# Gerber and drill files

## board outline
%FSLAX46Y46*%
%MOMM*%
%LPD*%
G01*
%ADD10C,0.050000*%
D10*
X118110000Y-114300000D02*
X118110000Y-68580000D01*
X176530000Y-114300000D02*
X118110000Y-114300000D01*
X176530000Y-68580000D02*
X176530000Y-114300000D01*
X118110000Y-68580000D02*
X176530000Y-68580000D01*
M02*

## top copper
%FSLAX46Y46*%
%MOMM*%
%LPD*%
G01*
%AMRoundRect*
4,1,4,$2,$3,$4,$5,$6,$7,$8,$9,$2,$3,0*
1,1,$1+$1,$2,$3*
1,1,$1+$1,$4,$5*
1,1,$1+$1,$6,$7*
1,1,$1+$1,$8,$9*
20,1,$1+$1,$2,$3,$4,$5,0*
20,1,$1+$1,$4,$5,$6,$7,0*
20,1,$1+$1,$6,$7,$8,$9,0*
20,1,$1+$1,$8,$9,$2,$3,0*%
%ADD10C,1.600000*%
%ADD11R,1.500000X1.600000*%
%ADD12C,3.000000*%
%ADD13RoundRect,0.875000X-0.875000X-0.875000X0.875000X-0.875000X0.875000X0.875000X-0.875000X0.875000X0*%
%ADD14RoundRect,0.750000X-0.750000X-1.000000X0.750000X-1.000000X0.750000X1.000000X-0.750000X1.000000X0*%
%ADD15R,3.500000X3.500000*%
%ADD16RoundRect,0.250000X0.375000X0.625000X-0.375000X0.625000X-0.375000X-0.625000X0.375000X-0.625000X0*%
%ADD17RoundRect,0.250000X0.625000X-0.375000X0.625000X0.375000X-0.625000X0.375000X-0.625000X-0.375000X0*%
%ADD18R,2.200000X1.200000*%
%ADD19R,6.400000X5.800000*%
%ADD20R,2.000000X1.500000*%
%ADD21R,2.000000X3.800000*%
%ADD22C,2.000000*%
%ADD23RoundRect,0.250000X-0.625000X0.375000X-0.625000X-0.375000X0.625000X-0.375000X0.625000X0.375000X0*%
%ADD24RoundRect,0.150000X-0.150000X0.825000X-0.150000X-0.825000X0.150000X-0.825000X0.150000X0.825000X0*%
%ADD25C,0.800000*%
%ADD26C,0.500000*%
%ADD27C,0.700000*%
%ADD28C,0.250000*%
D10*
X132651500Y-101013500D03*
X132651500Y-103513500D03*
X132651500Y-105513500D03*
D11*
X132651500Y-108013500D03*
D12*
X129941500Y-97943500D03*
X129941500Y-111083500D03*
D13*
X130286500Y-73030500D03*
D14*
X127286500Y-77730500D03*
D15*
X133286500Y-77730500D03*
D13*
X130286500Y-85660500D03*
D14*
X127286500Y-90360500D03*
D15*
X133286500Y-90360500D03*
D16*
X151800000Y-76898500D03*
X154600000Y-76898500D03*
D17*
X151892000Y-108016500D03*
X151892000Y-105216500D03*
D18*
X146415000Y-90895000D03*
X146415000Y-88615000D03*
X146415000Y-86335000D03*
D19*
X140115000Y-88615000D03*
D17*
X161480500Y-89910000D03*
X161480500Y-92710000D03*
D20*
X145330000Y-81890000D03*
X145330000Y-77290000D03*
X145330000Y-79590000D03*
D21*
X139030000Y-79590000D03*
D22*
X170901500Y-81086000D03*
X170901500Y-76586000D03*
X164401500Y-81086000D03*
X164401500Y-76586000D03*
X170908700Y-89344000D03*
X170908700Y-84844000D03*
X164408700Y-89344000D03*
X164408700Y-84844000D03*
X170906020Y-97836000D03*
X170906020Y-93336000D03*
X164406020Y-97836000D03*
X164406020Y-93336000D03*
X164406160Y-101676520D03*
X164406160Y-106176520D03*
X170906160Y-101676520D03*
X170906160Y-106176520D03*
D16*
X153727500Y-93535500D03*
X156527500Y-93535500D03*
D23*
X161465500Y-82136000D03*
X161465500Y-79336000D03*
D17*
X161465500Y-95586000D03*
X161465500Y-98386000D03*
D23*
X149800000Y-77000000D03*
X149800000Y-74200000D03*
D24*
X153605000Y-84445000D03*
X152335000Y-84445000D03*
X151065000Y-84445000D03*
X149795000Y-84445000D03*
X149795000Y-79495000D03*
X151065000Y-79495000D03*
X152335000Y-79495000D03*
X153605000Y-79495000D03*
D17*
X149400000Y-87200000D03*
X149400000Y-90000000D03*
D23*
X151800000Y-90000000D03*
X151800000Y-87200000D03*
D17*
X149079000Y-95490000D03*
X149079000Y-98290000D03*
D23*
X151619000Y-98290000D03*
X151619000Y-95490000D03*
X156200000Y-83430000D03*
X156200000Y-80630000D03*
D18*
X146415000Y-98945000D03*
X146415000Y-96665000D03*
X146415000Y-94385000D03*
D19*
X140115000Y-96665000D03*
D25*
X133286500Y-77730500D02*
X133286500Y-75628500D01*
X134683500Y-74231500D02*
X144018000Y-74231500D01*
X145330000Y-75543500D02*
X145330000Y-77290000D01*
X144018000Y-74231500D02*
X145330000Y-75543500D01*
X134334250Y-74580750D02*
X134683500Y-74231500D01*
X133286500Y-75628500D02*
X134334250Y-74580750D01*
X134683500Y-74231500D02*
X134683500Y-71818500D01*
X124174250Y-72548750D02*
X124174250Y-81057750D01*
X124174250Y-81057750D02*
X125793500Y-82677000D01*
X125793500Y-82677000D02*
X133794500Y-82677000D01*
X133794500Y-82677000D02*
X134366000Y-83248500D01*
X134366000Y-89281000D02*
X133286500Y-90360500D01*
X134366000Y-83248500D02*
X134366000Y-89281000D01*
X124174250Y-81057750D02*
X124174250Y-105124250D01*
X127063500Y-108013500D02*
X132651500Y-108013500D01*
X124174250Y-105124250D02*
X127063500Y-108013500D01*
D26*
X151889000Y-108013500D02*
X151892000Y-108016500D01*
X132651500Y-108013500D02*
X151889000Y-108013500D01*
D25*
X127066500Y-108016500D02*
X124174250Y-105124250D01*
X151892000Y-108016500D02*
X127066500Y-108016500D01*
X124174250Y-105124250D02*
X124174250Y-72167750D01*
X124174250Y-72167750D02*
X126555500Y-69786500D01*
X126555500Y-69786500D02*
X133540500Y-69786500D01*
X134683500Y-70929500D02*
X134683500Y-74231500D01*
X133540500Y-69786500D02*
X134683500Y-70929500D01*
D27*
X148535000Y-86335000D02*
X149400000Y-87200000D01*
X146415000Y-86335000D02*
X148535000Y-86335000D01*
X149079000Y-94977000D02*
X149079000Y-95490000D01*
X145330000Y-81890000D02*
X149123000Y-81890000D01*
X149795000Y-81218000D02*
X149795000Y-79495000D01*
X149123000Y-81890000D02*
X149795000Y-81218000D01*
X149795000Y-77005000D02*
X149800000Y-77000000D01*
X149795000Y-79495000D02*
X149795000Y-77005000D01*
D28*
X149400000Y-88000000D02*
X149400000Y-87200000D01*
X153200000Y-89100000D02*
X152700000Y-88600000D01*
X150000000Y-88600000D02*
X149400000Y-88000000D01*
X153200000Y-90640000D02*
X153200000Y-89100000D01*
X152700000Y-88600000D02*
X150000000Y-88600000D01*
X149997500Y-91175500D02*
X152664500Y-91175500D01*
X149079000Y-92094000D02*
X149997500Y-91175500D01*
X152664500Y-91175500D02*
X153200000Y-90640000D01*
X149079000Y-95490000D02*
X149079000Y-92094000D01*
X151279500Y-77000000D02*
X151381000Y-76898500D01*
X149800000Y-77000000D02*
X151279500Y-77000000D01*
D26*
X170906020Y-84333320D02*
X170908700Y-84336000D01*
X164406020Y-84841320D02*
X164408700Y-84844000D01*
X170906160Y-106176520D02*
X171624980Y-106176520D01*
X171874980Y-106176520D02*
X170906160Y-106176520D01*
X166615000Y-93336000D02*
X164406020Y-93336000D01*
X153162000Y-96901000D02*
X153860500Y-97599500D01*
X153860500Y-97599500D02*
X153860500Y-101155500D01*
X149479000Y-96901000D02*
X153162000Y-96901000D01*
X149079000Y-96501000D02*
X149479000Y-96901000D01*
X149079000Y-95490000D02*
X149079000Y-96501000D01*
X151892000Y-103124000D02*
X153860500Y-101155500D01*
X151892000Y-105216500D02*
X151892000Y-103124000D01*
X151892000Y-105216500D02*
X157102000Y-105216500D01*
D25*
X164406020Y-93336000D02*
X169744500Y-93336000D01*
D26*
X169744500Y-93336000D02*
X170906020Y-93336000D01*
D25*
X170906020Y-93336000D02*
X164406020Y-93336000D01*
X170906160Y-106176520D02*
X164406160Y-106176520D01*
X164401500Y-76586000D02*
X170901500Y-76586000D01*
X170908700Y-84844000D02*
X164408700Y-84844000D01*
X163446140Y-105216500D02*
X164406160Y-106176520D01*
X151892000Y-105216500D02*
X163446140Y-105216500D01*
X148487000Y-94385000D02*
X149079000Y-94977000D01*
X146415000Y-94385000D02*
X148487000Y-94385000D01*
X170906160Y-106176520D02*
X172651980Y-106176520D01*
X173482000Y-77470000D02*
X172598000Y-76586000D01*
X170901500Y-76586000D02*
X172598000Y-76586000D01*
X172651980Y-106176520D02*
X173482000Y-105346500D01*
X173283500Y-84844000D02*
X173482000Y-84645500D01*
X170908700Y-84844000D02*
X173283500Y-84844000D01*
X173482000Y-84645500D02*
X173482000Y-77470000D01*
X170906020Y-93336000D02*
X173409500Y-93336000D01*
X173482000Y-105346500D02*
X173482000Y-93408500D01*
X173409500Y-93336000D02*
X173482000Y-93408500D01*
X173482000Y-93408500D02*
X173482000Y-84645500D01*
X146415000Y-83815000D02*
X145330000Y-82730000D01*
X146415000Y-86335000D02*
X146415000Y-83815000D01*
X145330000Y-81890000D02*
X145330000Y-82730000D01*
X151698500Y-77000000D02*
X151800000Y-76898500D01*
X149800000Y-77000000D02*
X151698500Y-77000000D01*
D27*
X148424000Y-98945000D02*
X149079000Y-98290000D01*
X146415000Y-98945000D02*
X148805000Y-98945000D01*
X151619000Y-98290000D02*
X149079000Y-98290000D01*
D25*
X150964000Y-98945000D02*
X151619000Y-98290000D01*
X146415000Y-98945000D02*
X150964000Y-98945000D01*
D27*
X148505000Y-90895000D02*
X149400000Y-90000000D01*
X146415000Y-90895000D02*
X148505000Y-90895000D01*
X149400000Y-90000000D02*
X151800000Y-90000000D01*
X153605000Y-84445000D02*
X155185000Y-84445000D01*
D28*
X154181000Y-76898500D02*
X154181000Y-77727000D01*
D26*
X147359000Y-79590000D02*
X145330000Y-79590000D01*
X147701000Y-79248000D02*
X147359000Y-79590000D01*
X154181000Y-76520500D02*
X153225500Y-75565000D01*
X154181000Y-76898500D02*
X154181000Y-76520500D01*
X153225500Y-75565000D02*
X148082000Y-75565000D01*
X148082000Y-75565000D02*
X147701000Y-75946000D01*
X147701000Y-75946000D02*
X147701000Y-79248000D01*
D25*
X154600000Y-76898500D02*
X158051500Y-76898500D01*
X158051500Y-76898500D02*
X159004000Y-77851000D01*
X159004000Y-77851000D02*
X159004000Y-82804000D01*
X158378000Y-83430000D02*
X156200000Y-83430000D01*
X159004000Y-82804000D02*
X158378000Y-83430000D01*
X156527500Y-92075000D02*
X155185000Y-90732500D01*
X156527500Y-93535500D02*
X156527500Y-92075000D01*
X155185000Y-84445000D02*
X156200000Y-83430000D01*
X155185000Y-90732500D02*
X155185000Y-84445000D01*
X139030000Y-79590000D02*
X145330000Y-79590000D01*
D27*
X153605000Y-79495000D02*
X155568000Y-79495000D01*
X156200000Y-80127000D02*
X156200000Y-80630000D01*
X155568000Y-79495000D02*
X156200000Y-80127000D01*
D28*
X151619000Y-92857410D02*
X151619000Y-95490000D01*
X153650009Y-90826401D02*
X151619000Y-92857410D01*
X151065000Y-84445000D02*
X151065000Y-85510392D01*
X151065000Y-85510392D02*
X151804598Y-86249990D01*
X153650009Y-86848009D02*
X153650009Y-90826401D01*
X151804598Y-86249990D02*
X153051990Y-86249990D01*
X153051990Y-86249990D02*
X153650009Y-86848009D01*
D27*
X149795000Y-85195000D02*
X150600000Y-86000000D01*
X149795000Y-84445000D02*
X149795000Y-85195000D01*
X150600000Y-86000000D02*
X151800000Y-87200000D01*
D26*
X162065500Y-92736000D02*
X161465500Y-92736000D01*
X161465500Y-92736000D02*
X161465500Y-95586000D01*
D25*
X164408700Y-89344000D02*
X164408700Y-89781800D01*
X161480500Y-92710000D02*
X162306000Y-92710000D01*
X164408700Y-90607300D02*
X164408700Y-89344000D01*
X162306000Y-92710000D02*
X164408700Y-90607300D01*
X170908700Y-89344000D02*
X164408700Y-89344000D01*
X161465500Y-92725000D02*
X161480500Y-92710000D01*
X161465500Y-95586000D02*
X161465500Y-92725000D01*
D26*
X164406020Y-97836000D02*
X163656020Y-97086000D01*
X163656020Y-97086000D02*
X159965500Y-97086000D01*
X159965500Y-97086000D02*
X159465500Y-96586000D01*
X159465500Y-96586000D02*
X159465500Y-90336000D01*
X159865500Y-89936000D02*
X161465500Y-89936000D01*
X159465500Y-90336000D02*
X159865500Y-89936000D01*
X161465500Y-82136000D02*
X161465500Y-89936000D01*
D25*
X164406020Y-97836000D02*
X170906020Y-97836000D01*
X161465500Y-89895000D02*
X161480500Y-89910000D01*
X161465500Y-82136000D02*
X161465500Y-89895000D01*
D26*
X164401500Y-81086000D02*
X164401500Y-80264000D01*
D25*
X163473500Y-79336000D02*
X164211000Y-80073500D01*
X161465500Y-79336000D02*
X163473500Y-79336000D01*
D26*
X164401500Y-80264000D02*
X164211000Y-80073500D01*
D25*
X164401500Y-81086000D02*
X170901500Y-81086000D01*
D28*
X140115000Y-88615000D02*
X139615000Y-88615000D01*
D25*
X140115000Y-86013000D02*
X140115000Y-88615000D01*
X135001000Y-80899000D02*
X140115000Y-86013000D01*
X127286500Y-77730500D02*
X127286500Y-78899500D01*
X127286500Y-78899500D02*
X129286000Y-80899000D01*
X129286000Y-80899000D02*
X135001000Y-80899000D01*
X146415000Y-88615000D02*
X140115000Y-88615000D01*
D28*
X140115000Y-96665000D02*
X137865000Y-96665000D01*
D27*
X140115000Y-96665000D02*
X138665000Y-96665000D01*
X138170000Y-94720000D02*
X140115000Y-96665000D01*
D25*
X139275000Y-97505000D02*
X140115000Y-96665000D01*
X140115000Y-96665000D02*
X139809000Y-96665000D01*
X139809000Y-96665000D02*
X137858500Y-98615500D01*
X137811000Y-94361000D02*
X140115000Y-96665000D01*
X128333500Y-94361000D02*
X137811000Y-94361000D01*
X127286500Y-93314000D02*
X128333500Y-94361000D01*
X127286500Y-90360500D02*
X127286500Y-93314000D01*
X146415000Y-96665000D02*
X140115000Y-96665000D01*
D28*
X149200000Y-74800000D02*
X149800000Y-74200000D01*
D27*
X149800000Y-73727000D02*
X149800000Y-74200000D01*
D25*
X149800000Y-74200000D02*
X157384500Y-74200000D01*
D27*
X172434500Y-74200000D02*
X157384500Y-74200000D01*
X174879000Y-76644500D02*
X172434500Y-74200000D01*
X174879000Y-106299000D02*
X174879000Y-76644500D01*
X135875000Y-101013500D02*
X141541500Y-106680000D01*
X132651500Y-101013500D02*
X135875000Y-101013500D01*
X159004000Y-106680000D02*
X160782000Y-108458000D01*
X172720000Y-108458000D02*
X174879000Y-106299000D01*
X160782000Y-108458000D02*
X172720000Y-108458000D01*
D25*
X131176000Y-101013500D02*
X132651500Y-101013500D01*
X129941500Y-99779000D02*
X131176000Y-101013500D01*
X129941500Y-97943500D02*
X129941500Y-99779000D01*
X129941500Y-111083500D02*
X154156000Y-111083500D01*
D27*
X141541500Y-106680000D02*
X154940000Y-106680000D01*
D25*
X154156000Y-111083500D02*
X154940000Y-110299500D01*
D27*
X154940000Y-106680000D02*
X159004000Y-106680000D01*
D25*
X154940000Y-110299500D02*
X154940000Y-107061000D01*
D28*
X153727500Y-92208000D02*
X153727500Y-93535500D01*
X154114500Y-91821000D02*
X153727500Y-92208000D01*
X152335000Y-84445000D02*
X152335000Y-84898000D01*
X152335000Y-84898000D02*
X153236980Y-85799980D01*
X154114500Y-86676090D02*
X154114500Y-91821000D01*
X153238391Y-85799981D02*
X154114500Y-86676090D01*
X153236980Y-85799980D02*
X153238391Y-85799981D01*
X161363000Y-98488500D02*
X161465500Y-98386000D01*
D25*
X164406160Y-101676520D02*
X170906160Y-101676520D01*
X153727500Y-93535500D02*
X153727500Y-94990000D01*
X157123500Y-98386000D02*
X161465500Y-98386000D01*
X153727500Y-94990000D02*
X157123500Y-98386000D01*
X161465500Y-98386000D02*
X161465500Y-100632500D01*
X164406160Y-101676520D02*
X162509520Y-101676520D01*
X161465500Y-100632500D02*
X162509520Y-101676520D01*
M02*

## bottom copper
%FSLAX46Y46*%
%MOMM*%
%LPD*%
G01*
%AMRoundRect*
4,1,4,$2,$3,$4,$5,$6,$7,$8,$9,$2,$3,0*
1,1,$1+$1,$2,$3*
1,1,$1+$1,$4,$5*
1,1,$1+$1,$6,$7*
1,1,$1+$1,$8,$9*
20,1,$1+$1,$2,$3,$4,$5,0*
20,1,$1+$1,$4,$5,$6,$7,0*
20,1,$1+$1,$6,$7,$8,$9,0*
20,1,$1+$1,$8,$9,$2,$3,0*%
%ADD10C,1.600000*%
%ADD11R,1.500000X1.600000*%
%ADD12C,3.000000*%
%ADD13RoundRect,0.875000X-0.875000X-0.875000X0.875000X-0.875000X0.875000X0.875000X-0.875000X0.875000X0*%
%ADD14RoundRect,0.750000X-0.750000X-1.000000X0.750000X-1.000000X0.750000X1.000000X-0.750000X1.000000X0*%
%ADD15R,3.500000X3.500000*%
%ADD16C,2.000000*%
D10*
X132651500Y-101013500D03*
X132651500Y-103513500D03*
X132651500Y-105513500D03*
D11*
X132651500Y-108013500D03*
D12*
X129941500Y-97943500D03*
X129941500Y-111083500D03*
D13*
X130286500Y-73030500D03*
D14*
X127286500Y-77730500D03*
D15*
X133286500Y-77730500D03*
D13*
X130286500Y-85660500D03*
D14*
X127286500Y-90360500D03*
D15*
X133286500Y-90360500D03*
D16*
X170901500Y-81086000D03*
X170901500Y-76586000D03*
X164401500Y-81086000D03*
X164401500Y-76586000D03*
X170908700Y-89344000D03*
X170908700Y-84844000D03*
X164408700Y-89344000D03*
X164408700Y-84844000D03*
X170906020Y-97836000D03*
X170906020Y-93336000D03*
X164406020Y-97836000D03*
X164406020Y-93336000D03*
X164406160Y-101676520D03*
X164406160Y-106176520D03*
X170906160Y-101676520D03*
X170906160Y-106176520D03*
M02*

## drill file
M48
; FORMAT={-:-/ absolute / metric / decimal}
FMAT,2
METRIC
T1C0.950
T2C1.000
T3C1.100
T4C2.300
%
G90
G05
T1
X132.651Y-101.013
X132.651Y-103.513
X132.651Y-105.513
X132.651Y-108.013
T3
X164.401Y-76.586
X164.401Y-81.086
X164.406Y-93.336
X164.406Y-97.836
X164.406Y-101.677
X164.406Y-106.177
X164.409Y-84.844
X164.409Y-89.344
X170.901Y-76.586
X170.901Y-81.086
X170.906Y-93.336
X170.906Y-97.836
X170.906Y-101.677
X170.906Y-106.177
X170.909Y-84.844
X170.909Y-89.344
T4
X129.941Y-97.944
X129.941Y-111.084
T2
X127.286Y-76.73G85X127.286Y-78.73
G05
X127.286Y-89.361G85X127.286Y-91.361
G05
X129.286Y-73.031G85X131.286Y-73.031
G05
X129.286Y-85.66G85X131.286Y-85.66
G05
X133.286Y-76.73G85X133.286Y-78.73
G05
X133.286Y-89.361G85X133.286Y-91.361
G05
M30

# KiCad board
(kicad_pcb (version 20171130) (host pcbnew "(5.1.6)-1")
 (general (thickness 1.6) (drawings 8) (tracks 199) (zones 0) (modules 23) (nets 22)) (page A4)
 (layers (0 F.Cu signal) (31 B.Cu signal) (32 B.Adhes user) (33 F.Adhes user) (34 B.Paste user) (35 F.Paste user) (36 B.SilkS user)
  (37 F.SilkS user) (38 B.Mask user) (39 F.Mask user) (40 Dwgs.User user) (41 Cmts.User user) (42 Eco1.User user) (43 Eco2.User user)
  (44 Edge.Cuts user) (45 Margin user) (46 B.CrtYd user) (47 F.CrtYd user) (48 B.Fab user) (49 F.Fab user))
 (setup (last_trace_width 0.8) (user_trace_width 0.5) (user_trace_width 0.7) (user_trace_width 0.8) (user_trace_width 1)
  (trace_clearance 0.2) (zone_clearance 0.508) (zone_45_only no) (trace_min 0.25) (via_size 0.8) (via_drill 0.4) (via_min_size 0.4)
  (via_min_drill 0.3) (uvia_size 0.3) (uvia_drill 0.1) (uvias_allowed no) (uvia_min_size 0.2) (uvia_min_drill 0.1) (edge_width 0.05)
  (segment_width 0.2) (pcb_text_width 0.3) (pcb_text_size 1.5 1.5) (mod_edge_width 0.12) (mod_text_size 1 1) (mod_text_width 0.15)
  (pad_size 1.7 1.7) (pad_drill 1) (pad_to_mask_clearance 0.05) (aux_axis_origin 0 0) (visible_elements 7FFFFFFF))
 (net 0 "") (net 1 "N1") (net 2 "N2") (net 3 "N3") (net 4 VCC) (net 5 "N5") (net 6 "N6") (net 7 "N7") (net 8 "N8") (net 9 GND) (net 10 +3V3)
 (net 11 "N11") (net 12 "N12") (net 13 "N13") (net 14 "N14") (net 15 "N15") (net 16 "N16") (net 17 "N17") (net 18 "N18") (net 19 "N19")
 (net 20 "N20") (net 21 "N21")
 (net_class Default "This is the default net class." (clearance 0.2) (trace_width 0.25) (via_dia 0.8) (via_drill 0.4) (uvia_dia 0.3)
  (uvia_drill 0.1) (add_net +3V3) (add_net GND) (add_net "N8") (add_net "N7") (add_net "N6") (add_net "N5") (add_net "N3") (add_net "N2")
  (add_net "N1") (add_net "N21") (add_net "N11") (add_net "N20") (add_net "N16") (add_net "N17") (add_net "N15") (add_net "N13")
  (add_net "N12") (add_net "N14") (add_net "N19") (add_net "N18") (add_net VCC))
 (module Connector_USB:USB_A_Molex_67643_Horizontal (layer B.Cu) (at 132.6515 108.0135 90)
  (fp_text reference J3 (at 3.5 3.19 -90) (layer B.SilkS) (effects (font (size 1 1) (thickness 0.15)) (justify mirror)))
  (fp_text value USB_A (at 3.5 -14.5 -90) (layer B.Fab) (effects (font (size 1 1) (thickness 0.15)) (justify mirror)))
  (pad 4 thru_hole circle (at 7 0 90) (size 1.6 1.6) (drill 0.95) (layers *.Cu *.Mask) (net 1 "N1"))
  (pad 3 thru_hole circle (at 4.5 0 90) (size 1.6 1.6) (drill 0.95) (layers *.Cu *.Mask) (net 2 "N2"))
  (pad 2 thru_hole circle (at 2.5 0 90) (size 1.6 1.6) (drill 0.95) (layers *.Cu *.Mask) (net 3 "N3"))
  (pad 1 thru_hole rect (at 0 0 90) (size 1.6 1.5) (drill 0.95) (layers *.Cu *.Mask) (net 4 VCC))
  (pad 5 thru_hole circle (at 10.07 -2.71 90) (size 3 3) (drill 2.3) (layers *.Cu *.Mask) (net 1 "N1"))
  (pad 5 thru_hole circle (at -3.07 -2.71 90) (size 3 3) (drill 2.3) (layers *.Cu *.Mask) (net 1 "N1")))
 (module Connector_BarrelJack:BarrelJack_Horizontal (layer B.Cu) (at 133.2865 77.7305)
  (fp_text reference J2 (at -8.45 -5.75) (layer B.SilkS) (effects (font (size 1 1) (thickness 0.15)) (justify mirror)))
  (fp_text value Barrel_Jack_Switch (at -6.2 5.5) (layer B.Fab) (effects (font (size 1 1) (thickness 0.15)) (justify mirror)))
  (pad 3 thru_hole roundrect (at -3 -4.7) (size 3.5 3.5) (drill oval 3 1) (layers *.Cu *.Mask) (roundrect_rratio 0.25) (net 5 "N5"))
  (pad 2 thru_hole roundrect (at -6 0) (size 3 3.5) (drill oval 1 3) (layers *.Cu *.Mask) (roundrect_rratio 0.25) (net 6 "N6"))
  (pad 1 thru_hole rect (at 0 0) (size 3.5 3.5) (drill oval 1 3) (layers *.Cu *.Mask) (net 4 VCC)))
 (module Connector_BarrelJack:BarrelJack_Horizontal (layer B.Cu) (at 133.2865 90.3605)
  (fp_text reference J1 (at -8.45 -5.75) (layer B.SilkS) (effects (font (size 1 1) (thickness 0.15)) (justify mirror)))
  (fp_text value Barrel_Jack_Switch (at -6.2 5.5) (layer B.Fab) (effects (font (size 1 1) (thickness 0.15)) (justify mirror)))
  (pad 3 thru_hole roundrect (at -3 -4.7) (size 3.5 3.5) (drill oval 3 1) (layers *.Cu *.Mask) (roundrect_rratio 0.25) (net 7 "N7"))
  (pad 2 thru_hole roundrect (at -6 0) (size 3 3.5) (drill oval 1 3) (layers *.Cu *.Mask) (roundrect_rratio 0.25) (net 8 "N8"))
  (pad 1 thru_hole rect (at 0 0) (size 3.5 3.5) (drill oval 1 3) (layers *.Cu *.Mask) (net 4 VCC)))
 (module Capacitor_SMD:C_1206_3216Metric (layer F.Cu) (at 153.2 76.8985 180)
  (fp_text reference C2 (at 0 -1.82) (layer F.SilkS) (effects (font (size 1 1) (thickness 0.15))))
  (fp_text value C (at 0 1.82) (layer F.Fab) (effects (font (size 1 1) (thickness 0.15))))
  (pad 2 smd roundrect (at 1.4 0 180) (size 1.25 1.75) (layers F.Cu F.Paste F.Mask) (roundrect_rratio 0.2) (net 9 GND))
  (pad 1 smd roundrect (at -1.4 0 180) (size 1.25 1.75) (layers F.Cu F.Paste F.Mask) (roundrect_rratio 0.2) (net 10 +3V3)))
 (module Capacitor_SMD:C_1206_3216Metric (layer F.Cu) (at 151.892 106.6165 90)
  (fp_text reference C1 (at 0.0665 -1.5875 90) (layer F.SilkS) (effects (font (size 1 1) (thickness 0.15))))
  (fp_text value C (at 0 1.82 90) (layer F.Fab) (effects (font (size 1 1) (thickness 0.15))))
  (pad 1 smd roundrect (at -1.4 0 90) (size 1.25 1.75) (layers F.Cu F.Paste F.Mask) (roundrect_rratio 0.2) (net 4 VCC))
  (pad 2 smd roundrect (at 1.4 0 90) (size 1.25 1.75) (layers F.Cu F.Paste F.Mask) (roundrect_rratio 0.2) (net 9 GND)))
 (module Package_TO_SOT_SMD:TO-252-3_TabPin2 (layer F.Cu) (at 142.215 88.615 180)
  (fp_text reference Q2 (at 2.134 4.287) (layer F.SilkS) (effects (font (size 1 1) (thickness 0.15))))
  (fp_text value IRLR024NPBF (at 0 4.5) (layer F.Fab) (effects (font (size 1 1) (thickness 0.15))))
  (pad 1 smd rect (at -4.2 -2.28 180) (size 2.2 1.2) (layers F.Cu F.Paste F.Mask) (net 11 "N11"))
  (pad 2 smd rect (at -4.2 0 180) (size 2.2 1.2) (layers F.Cu F.Paste F.Mask) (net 6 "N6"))
  (pad 3 smd rect (at -4.2 2.28 180) (size 2.2 1.2) (layers F.Cu F.Paste F.Mask) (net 9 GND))
  (pad 2 smd rect (at 2.1 0 180) (size 6.4 5.8) (layers F.Cu F.Mask) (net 6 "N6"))
  (pad "" smd rect (at 3.775 1.525 180) (size 3.05 2.75) (layers F.Paste))
  (pad "" smd rect (at 0.425 -1.525 180) (size 3.05 2.75) (layers F.Paste))
  (pad "" smd rect (at 3.775 -1.525 180) (size 3.05 2.75) (layers F.Paste))
  (pad "" smd rect (at 0.425 1.525 180) (size 3.05 2.75) (layers F.Paste)))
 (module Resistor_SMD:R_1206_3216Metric (layer F.Cu) (at 161.4805 91.31 90)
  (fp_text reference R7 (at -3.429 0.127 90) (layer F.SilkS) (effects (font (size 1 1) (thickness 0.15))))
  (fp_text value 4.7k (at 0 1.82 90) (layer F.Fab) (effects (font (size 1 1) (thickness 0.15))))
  (pad 2 smd roundrect (at 1.4 0 90) (size 1.25 1.75) (layers F.Cu F.Paste F.Mask) (roundrect_rratio 0.2) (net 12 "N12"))
  (pad 1 smd roundrect (at -1.4 0 90) (size 1.25 1.75) (layers F.Cu F.Paste F.Mask) (roundrect_rratio 0.2) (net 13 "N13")))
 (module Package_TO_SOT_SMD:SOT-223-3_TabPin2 (layer F.Cu) (at 142.18 79.59 180)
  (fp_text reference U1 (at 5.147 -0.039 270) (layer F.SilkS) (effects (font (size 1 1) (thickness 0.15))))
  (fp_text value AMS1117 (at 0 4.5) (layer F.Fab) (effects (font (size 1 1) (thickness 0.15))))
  (pad 1 smd rect (at -3.15 -2.3 180) (size 2 1.5) (layers F.Cu F.Paste F.Mask) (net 9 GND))
  (pad 3 smd rect (at -3.15 2.3 180) (size 2 1.5) (layers F.Cu F.Paste F.Mask) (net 4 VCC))
  (pad 2 smd rect (at -3.15 0 180) (size 2 1.5) (layers F.Cu F.Paste F.Mask) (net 10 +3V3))
  (pad 2 smd rect (at 3.15 0 180) (size 2 3.8) (layers F.Cu F.Paste F.Mask) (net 10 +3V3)))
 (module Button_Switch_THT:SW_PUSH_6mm (layer B.Cu) (at 164.4015 81.086)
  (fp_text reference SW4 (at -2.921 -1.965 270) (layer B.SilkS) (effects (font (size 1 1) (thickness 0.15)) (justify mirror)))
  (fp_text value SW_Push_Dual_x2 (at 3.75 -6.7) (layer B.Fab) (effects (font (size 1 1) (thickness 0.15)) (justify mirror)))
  (pad 1 thru_hole circle (at 6.5 0 270) (size 2 2) (drill 1.1) (layers *.Cu *.Mask) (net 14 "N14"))
  (pad 2 thru_hole circle (at 6.5 -4.5 270) (size 2 2) (drill 1.1) (layers *.Cu *.Mask) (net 9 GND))
  (pad 1 thru_hole circle (at 0 0 270) (size 2 2) (drill 1.1) (layers *.Cu *.Mask) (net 14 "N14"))
  (pad 2 thru_hole circle (at 0 -4.5 270) (size 2 2) (drill 1.1) (layers *.Cu *.Mask) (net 9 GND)))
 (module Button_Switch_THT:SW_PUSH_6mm (layer B.Cu) (at 164.4087 89.344)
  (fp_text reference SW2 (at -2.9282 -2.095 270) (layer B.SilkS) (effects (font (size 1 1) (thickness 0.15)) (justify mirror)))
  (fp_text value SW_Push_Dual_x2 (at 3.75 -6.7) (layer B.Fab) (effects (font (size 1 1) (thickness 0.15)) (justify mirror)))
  (pad 1 thru_hole circle (at 6.5 0 270) (size 2 2) (drill 1.1) (layers *.Cu *.Mask) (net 13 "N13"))
  (pad 2 thru_hole circle (at 6.5 -4.5 270) (size 2 2) (drill 1.1) (layers *.Cu *.Mask) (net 9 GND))
  (pad 1 thru_hole circle (at 0 0 270) (size 2 2) (drill 1.1) (layers *.Cu *.Mask) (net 13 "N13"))
  (pad 2 thru_hole circle (at 0 -4.5 270) (size 2 2) (drill 1.1) (layers *.Cu *.Mask) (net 9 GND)))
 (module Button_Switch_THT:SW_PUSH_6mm (layer B.Cu) (at 164.40602 97.836)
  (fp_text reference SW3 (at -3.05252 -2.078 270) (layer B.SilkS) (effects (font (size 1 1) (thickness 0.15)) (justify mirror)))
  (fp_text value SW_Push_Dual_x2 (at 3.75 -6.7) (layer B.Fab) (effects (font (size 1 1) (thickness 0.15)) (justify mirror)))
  (pad 1 thru_hole circle (at 6.5 0 270) (size 2 2) (drill 1.1) (layers *.Cu *.Mask) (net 12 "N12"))
  (pad 2 thru_hole circle (at 6.5 -4.5 270) (size 2 2) (drill 1.1) (layers *.Cu *.Mask) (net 9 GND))
  (pad 1 thru_hole circle (at 0 0 270) (size 2 2) (drill 1.1) (layers *.Cu *.Mask) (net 12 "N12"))
  (pad 2 thru_hole circle (at 0 -4.5 270) (size 2 2) (drill 1.1) (layers *.Cu *.Mask) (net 9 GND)))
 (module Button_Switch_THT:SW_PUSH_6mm (layer B.Cu) (at 170.90616 101.67652 180)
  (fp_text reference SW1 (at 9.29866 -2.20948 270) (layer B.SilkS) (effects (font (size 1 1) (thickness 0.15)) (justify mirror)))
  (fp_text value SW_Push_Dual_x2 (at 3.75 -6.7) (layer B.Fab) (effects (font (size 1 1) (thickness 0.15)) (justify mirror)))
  (pad 1 thru_hole circle (at 6.5 0 90) (size 2 2) (drill 1.1) (layers *.Cu *.Mask) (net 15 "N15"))
  (pad 2 thru_hole circle (at 6.5 -4.5 90) (size 2 2) (drill 1.1) (layers *.Cu *.Mask) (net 9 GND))
  (pad 1 thru_hole circle (at 0 0 90) (size 2 2) (drill 1.1) (layers *.Cu *.Mask) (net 15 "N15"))
  (pad 2 thru_hole circle (at 0 -4.5 90) (size 2 2) (drill 1.1) (layers *.Cu *.Mask) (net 9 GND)))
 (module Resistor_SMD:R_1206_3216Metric (layer F.Cu) (at 155.1275 93.5355 180)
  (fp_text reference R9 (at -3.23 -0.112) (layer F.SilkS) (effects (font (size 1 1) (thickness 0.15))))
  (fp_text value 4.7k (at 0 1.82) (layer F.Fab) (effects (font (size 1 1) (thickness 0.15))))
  (pad 2 smd roundrect (at 1.4 0 180) (size 1.25 1.75) (layers F.Cu F.Paste F.Mask) (roundrect_rratio 0.2) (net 15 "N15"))
  (pad 1 smd roundrect (at -1.4 0 180) (size 1.25 1.75) (layers F.Cu F.Paste F.Mask) (roundrect_rratio 0.2) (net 10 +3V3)))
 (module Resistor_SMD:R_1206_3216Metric (layer F.Cu) (at 161.4655 80.736 270)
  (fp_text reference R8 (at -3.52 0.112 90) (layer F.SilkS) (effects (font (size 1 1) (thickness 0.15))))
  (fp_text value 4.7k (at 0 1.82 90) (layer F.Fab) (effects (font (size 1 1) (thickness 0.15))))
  (pad 2 smd roundrect (at 1.4 0 270) (size 1.25 1.75) (layers F.Cu F.Paste F.Mask) (roundrect_rratio 0.2) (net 12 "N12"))
  (pad 1 smd roundrect (at -1.4 0 270) (size 1.25 1.75) (layers F.Cu F.Paste F.Mask) (roundrect_rratio 0.2) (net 14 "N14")))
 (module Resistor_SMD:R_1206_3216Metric (layer F.Cu) (at 161.4655 96.986 90)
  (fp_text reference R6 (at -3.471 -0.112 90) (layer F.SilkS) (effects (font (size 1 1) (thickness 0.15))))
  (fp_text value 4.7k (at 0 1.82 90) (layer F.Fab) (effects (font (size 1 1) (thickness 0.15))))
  (pad 2 smd roundrect (at 1.4 0 90) (size 1.25 1.75) (layers F.Cu F.Paste F.Mask) (roundrect_rratio 0.2) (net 13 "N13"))
  (pad 1 smd roundrect (at -1.4 0 90) (size 1.25 1.75) (layers F.Cu F.Paste F.Mask) (roundrect_rratio 0.2) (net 15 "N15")))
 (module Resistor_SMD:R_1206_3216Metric (layer F.Cu) (at 149.8 75.6 270)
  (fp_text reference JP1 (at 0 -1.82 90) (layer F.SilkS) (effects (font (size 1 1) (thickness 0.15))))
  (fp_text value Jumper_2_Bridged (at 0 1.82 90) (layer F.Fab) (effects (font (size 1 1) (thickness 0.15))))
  (pad 2 smd roundrect (at 1.4 0 270) (size 1.25 1.75) (layers F.Cu F.Paste F.Mask) (roundrect_rratio 0.2) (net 9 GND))
  (pad 1 smd roundrect (at -1.4 0 270) (size 1.25 1.75) (layers F.Cu F.Paste F.Mask) (roundrect_rratio 0.2) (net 1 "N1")))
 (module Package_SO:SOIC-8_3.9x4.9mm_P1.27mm (layer F.Cu) (at 151.7 81.97 270)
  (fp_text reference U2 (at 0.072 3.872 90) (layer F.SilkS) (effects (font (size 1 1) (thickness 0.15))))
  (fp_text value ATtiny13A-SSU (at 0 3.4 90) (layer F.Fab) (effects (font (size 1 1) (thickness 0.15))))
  (pad 8 smd roundrect (at 2.475 -1.905 270) (size 1.95 0.6) (layers F.Cu F.Paste F.Mask) (roundrect_rratio 0.25) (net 10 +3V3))
  (pad 7 smd roundrect (at 2.475 -0.635 270) (size 1.95 0.6) (layers F.Cu F.Paste F.Mask) (roundrect_rratio 0.25) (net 15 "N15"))
  (pad 6 smd roundrect (at 2.475 0.635 270) (size 1.95 0.6) (layers F.Cu F.Paste F.Mask) (roundrect_rratio 0.25) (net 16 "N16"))
  (pad 5 smd roundrect (at 2.475 1.905 270) (size 1.95 0.6) (layers F.Cu F.Paste F.Mask) (roundrect_rratio 0.25) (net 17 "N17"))
  (pad 4 smd roundrect (at -2.475 1.905 270) (size 1.95 0.6) (layers F.Cu F.Paste F.Mask) (roundrect_rratio 0.25) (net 9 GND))
  (pad 3 smd roundrect (at -2.475 0.635 270) (size 1.95 0.6) (layers F.Cu F.Paste F.Mask) (roundrect_rratio 0.25) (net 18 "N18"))
  (pad 2 smd roundrect (at -2.475 -0.635 270) (size 1.95 0.6) (layers F.Cu F.Paste F.Mask) (roundrect_rratio 0.25) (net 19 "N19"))
  (pad 1 smd roundrect (at -2.475 -1.905 270) (size 1.95 0.6) (layers F.Cu F.Paste F.Mask) (roundrect_rratio 0.25) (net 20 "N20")))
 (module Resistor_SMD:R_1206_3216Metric (layer F.Cu) (at 149.4 88.6 90)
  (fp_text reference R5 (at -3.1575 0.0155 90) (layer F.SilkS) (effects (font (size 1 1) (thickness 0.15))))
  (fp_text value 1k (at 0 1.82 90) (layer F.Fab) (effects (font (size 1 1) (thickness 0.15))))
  (pad 2 smd roundrect (at 1.4 0 90) (size 1.25 1.75) (layers F.Cu F.Paste F.Mask) (roundrect_rratio 0.2) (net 9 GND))
  (pad 1 smd roundrect (at -1.4 0 90) (size 1.25 1.75) (layers F.Cu F.Paste F.Mask) (roundrect_rratio 0.2) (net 11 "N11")))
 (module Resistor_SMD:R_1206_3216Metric (layer F.Cu) (at 151.8 88.6 270)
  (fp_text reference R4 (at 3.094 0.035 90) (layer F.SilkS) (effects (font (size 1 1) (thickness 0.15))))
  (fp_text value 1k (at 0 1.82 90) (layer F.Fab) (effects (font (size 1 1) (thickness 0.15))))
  (pad 2 smd roundrect (at 1.4 0 270) (size 1.25 1.75) (layers F.Cu F.Paste F.Mask) (roundrect_rratio 0.2) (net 11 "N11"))
  (pad 1 smd roundrect (at -1.4 0 270) (size 1.25 1.75) (layers F.Cu F.Paste F.Mask) (roundrect_rratio 0.2) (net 17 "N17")))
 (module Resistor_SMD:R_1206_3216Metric (layer F.Cu) (at 149.079 96.89 90)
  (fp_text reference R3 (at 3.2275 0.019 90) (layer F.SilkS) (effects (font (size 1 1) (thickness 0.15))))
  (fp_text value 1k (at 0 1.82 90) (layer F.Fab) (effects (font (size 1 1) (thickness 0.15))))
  (pad 2 smd roundrect (at 1.4 0 90) (size 1.25 1.75) (layers F.Cu F.Paste F.Mask) (roundrect_rratio 0.2) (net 9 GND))
  (pad 1 smd roundrect (at -1.4 0 90) (size 1.25 1.75) (layers F.Cu F.Paste F.Mask) (roundrect_rratio 0.2) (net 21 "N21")))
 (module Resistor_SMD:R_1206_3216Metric (layer F.Cu) (at 151.619 96.89 270)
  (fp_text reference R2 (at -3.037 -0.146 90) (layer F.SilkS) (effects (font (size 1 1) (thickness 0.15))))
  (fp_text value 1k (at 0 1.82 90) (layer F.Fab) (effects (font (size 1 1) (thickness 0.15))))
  (pad 2 smd roundrect (at 1.4 0 270) (size 1.25 1.75) (layers F.Cu F.Paste F.Mask) (roundrect_rratio 0.2) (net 21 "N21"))
  (pad 1 smd roundrect (at -1.4 0 270) (size 1.25 1.75) (layers F.Cu F.Paste F.Mask) (roundrect_rratio 0.2) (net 16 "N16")))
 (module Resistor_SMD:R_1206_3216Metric (layer F.Cu) (at 156.2 82.03 270)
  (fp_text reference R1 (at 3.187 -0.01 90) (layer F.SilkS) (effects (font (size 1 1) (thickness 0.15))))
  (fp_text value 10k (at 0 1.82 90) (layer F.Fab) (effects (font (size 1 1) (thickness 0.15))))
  (pad 2 smd roundrect (at 1.4 0 270) (size 1.25 1.75) (layers F.Cu F.Paste F.Mask) (roundrect_rratio 0.2) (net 10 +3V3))
  (pad 1 smd roundrect (at -1.4 0 270) (size 1.25 1.75) (layers F.Cu F.Paste F.Mask) (roundrect_rratio 0.2) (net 20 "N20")))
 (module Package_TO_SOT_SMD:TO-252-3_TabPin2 (layer F.Cu) (at 142.215 96.665 180)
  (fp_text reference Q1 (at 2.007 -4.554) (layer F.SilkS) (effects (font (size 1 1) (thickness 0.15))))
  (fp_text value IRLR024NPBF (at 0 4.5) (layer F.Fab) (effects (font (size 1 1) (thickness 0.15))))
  (pad 1 smd rect (at -4.2 -2.28 180) (size 2.2 1.2) (layers F.Cu F.Paste F.Mask) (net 21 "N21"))
  (pad 2 smd rect (at -4.2 0 180) (size 2.2 1.2) (layers F.Cu F.Paste F.Mask) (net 8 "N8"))
  (pad 3 smd rect (at -4.2 2.28 180) (size 2.2 1.2) (layers F.Cu F.Paste F.Mask) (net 9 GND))
  (pad 2 smd rect (at 2.1 0 180) (size 6.4 5.8) (layers F.Cu F.Mask) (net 8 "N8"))
  (pad "" smd rect (at 3.775 1.525 180) (size 3.05 2.75) (layers F.Paste))
  (pad "" smd rect (at 0.425 -1.525 180) (size 3.05 2.75) (layers F.Paste))
  (pad "" smd rect (at 3.775 -1.525 180) (size 3.05 2.75) (layers F.Paste))
  (pad "" smd rect (at 0.425 1.525 180) (size 3.05 2.75) (layers F.Paste)))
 (gr_line (start 118.11 114.3) (end 118.11 68.58) (layer Edge.Cuts) (width 0.05))
 (gr_line (start 176.53 114.3) (end 118.11 114.3) (layer Edge.Cuts) (width 0.05))
 (gr_line (start 176.53 68.58) (end 176.53 114.3) (layer Edge.Cuts) (width 0.05))
 (gr_line (start 118.11 68.58) (end 176.53 68.58) (layer Edge.Cuts) (width 0.05))
 (segment (start 133.2865 77.7305) (end 133.2865 75.6285) (width 0.8) (layer F.Cu) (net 4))
 (segment (start 134.6835 74.2315) (end 144.018 74.2315) (width 0.8) (layer F.Cu) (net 4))
 (segment (start 145.33 75.5435) (end 145.33 77.29) (width 0.8) (layer F.Cu) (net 4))
 (segment (start 144.018 74.2315) (end 145.33 75.5435) (width 0.8) (layer F.Cu) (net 4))
 (segment (start 134.33425 74.58075) (end 134.6835 74.2315) (width 0.8) (layer F.Cu) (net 4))
 (segment (start 133.2865 75.6285) (end 134.33425 74.58075) (width 0.8) (layer F.Cu) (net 4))
 (segment (start 134.6835 74.2315) (end 134.6835 71.8185) (width 0.8) (layer F.Cu) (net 4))
 (segment (start 124.17425 72.54875) (end 124.17425 81.05775) (width 0.8) (layer F.Cu) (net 4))
 (segment (start 124.17425 81.05775) (end 125.7935 82.677) (width 0.8) (layer F.Cu) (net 4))
 (segment (start 125.7935 82.677) (end 133.7945 82.677) (width 0.8) (layer F.Cu) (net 4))
 (segment (start 133.7945 82.677) (end 134.366 83.2485) (width 0.8) (layer F.Cu) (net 4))
 (segment (start 134.366 89.281) (end 133.2865 90.3605) (width 0.8) (layer F.Cu) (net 4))
 (segment (start 134.366 83.2485) (end 134.366 89.281) (width 0.8) (layer F.Cu) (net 4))
 (segment (start 124.17425 81.05775) (end 124.17425 105.12425) (width 0.8) (layer F.Cu) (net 4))
 (segment (start 127.0635 108.0135) (end 132.6515 108.0135) (width 0.8) (layer F.Cu) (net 4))
 (segment (start 124.17425 105.12425) (end 127.0635 108.0135) (width 0.8) (layer F.Cu) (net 4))
 (segment (start 151.889 108.0135) (end 151.892 108.0165) (width 0.5) (layer F.Cu) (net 4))
 (segment (start 132.6515 108.0135) (end 151.889 108.0135) (width 0.5) (layer F.Cu) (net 4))
 (segment (start 127.0665 108.0165) (end 124.17425 105.12425) (width 0.8) (layer F.Cu) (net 4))
 (segment (start 151.892 108.0165) (end 127.0665 108.0165) (width 0.8) (layer F.Cu) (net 4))
 (segment (start 124.17425 105.12425) (end 124.17425 72.16775) (width 0.8) (layer F.Cu) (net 4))
 (segment (start 124.17425 72.16775) (end 126.5555 69.7865) (width 0.8) (layer F.Cu) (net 4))
 (segment (start 126.5555 69.7865) (end 133.5405 69.7865) (width 0.8) (layer F.Cu) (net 4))
 (segment (start 134.6835 70.9295) (end 134.6835 74.2315) (width 0.8) (layer F.Cu) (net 4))
 (segment (start 133.5405 69.7865) (end 134.6835 70.9295) (width 0.8) (layer F.Cu) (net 4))
 (segment (start 148.535 86.335) (end 149.4 87.2) (width 0.7) (layer F.Cu) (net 9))
 (segment (start 146.415 86.335) (end 148.535 86.335) (width 0.7) (layer F.Cu) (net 9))
 (segment (start 149.079 94.977) (end 149.079 95.49) (width 0.7) (layer F.Cu) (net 9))
 (segment (start 145.33 81.89) (end 149.123 81.89) (width 0.7) (layer F.Cu) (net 9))
 (segment (start 149.795 81.218) (end 149.795 79.495) (width 0.7) (layer F.Cu) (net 9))
 (segment (start 149.123 81.89) (end 149.795 81.218) (width 0.7) (layer F.Cu) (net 9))
 (segment (start 149.795 77.005) (end 149.8 77) (width 0.7) (layer F.Cu) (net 9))
 (segment (start 149.795 79.495) (end 149.795 77.005) (width 0.7) (layer F.Cu) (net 9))
 (segment (start 149.4 88) (end 149.4 87.2) (width 0.25) (layer F.Cu) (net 9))
 (segment (start 153.2 89.1) (end 152.7 88.6) (width 0.25) (layer F.Cu) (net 9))
 (segment (start 150 88.6) (end 149.4 88) (width 0.25) (layer F.Cu) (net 9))
 (segment (start 153.2 90.64) (end 153.2 89.1) (width 0.25) (layer F.Cu) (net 9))
 (segment (start 152.7 88.6) (end 150 88.6) (width 0.25) (layer F.Cu) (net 9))
 (segment (start 149.9975 91.1755) (end 152.6645 91.1755) (width 0.25) (layer F.Cu) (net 9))
 (segment (start 149.079 92.094) (end 149.9975 91.1755) (width 0.25) (layer F.Cu) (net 9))
 (segment (start 152.6645 91.1755) (end 153.2 90.64) (width 0.25) (layer F.Cu) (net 9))
 (segment (start 149.079 95.49) (end 149.079 92.094) (width 0.25) (layer F.Cu) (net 9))
 (segment (start 151.2795 77) (end 151.381 76.8985) (width 0.25) (layer F.Cu) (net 9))
 (segment (start 149.8 77) (end 151.2795 77) (width 0.25) (layer F.Cu) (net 9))
 (segment (start 170.90602 84.33332) (end 170.9087 84.336) (width 0.5) (layer F.Cu) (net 9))
 (segment (start 164.40602 84.84132) (end 164.4087 84.844) (width 0.5) (layer F.Cu) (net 9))
 (segment (start 170.90616 106.17652) (end 171.62498 106.17652) (width 0.5) (layer F.Cu) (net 9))
 (segment (start 171.87498 106.17652) (end 170.90616 106.17652) (width 0.5) (layer F.Cu) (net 9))
 (segment (start 166.615 93.336) (end 164.40602 93.336) (width 0.5) (layer F.Cu) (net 9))
 (segment (start 153.162 96.901) (end 153.8605 97.5995) (width 0.5) (layer F.Cu) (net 9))
 (segment (start 153.8605 97.5995) (end 153.8605 101.1555) (width 0.5) (layer F.Cu) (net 9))
 (segment (start 149.479 96.901) (end 153.162 96.901) (width 0.5) (layer F.Cu) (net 9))
 (segment (start 149.079 96.501) (end 149.479 96.901) (width 0.5) (layer F.Cu) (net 9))
 (segment (start 149.079 95.49) (end 149.079 96.501) (width 0.5) (layer F.Cu) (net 9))
 (segment (start 151.892 103.124) (end 153.8605 101.1555) (width 0.5) (layer F.Cu) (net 9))
 (segment (start 151.892 105.2165) (end 151.892 103.124) (width 0.5) (layer F.Cu) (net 9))
 (segment (start 151.892 105.2165) (end 157.102 105.2165) (width 0.5) (layer F.Cu) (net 9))
 (segment (start 164.40602 93.336) (end 169.7445 93.336) (width 0.8) (layer F.Cu) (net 9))
 (segment (start 169.7445 93.336) (end 170.90602 93.336) (width 0.5) (layer F.Cu) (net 9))
 (segment (start 170.90602 93.336) (end 164.40602 93.336) (width 0.8) (layer F.Cu) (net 9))
 (segment (start 170.90616 106.17652) (end 164.40616 106.17652) (width 0.8) (layer F.Cu) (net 9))
 (segment (start 164.4015 76.586) (end 170.9015 76.586) (width 0.8) (layer F.Cu) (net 9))
 (segment (start 170.9087 84.844) (end 164.4087 84.844) (width 0.8) (layer F.Cu) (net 9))
 (segment (start 163.44614 105.2165) (end 164.40616 106.17652) (width 0.8) (layer F.Cu) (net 9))
 (segment (start 151.892 105.2165) (end 163.44614 105.2165) (width 0.8) (layer F.Cu) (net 9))
 (segment (start 148.487 94.385) (end 149.079 94.977) (width 0.8) (layer F.Cu) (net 9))
 (segment (start 146.415 94.385) (end 148.487 94.385) (width 0.8) (layer F.Cu) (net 9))
 (segment (start 170.90616 106.17652) (end 172.65198 106.17652) (width 0.8) (layer F.Cu) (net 9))
 (segment (start 173.482 77.47) (end 172.598 76.586) (width 0.8) (layer F.Cu) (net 9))
 (segment (start 170.9015 76.586) (end 172.598 76.586) (width 0.8) (layer F.Cu) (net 9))
 (segment (start 172.65198 106.17652) (end 173.482 105.3465) (width 0.8) (layer F.Cu) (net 9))
 (segment (start 173.2835 84.844) (end 173.482 84.6455) (width 0.8) (layer F.Cu) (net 9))
 (segment (start 170.9087 84.844) (end 173.2835 84.844) (width 0.8) (layer F.Cu) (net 9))
 (segment (start 173.482 84.6455) (end 173.482 77.47) (width 0.8) (layer F.Cu) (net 9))
 (segment (start 170.90602 93.336) (end 173.4095 93.336) (width 0.8) (layer F.Cu) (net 9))
 (segment (start 173.482 105.3465) (end 173.482 93.4085) (width 0.8) (layer F.Cu) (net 9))
 (segment (start 173.4095 93.336) (end 173.482 93.4085) (width 0.8) (layer F.Cu) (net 9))
 (segment (start 173.482 93.4085) (end 173.482 84.6455) (width 0.8) (layer F.Cu) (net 9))
 (segment (start 146.415 83.815) (end 145.33 82.73) (width 0.8) (layer F.Cu) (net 9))
 (segment (start 146.415 86.335) (end 146.415 83.815) (width 0.8) (layer F.Cu) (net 9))
 (segment (start 145.33 81.89) (end 145.33 82.73) (width 0.8) (layer F.Cu) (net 9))
 (segment (start 151.6985 77) (end 151.8 76.8985) (width 0.8) (layer F.Cu) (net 9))
 (segment (start 149.8 77) (end 151.6985 77) (width 0.8) (layer F.Cu) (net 9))
 (segment (start 148.424 98.945) (end 149.079 98.29) (width 0.7) (layer F.Cu) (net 21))
 (segment (start 146.415 98.945) (end 148.805 98.945) (width 0.7) (layer F.Cu) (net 21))
 (segment (start 151.619 98.29) (end 149.079 98.29) (width 0.7) (layer F.Cu) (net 21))
 (segment (start 150.964 98.945) (end 151.619 98.29) (width 0.8) (layer F.Cu) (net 21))
 (segment (start 146.415 98.945) (end 150.964 98.945) (width 0.8) (layer F.Cu) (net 21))
 (segment (start 148.505 90.895) (end 149.4 90) (width 0.7) (layer F.Cu) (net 11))
 (segment (start 146.415 90.895) (end 148.505 90.895) (width 0.7) (layer F.Cu) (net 11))
 (segment (start 149.4 90) (end 151.8 90) (width 0.7) (layer F.Cu) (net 11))
 (segment (start 153.605 84.445) (end 155.185 84.445) (width 0.7) (layer F.Cu) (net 10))
 (segment (start 154.181 76.8985) (end 154.181 77.727) (width 0.25) (layer F.Cu) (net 10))
 (segment (start 147.359 79.59) (end 145.33 79.59) (width 0.5) (layer F.Cu) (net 10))
 (segment (start 147.701 79.248) (end 147.359 79.59) (width 0.5) (layer F.Cu) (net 10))
 (segment (start 154.181 76.5205) (end 153.2255 75.565) (width 0.5) (layer F.Cu) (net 10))
 (segment (start 154.181 76.8985) (end 154.181 76.5205) (width 0.5) (layer F.Cu) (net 10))
 (segment (start 153.2255 75.565) (end 148.082 75.565) (width 0.5) (layer F.Cu) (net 10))
 (segment (start 148.082 75.565) (end 147.701 75.946) (width 0.5) (layer F.Cu) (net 10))
 (segment (start 147.701 75.946) (end 147.701 79.248) (width 0.5) (layer F.Cu) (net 10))
 (segment (start 154.6 76.8985) (end 158.0515 76.8985) (width 0.8) (layer F.Cu) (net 10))
 (segment (start 158.0515 76.8985) (end 159.004 77.851) (width 0.8) (layer F.Cu) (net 10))
 (segment (start 159.004 77.851) (end 159.004 82.804) (width 0.8) (layer F.Cu) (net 10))
 (segment (start 158.378 83.43) (end 156.2 83.43) (width 0.8) (layer F.Cu) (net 10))
 (segment (start 159.004 82.804) (end 158.378 83.43) (width 0.8) (layer F.Cu) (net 10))
 (segment (start 156.5275 92.075) (end 155.185 90.7325) (width 0.8) (layer F.Cu) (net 10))
 (segment (start 156.5275 93.5355) (end 156.5275 92.075) (width 0.8) (layer F.Cu) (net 10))
 (segment (start 155.185 84.445) (end 156.2 83.43) (width 0.8) (layer F.Cu) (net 10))
 (segment (start 155.185 90.7325) (end 155.185 84.445) (width 0.8) (layer F.Cu) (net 10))
 (segment (start 139.03 79.59) (end 145.33 79.59) (width 0.8) (layer F.Cu) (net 10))
 (segment (start 153.605 79.495) (end 155.568 79.495) (width 0.7) (layer F.Cu) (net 20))
 (segment (start 156.2 80.127) (end 156.2 80.63) (width 0.7) (layer F.Cu) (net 20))
 (segment (start 155.568 79.495) (end 156.2 80.127) (width 0.7) (layer F.Cu) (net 20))
 (segment (start 151.619 92.85741) (end 151.619 95.49) (width 0.25) (layer F.Cu) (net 16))
 (segment (start 153.650009 90.826401) (end 151.619 92.85741) (width 0.25) (layer F.Cu) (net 16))
 (segment (start 151.065 84.445) (end 151.065 85.510392) (width 0.25) (layer F.Cu) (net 16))
 (segment (start 151.065 85.510392) (end 151.804598 86.24999) (width 0.25) (layer F.Cu) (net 16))
 (segment (start 153.650009 86.848009) (end 153.650009 90.826401) (width 0.25) (layer F.Cu) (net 16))
 (segment (start 151.804598 86.24999) (end 153.05199 86.24999) (width 0.25) (layer F.Cu) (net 16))
 (segment (start 153.05199 86.24999) (end 153.650009 86.848009) (width 0.25) (layer F.Cu) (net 16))
 (segment (start 149.795 85.195) (end 150.6 86) (width 0.7) (layer F.Cu) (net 17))
 (segment (start 149.795 84.445) (end 149.795 85.195) (width 0.7) (layer F.Cu) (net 17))
 (segment (start 150.6 86) (end 151.8 87.2) (width 0.7) (layer F.Cu) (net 17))
 (segment (start 162.0655 92.736) (end 161.4655 92.736) (width 0.5) (layer F.Cu) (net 13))
 (segment (start 161.4655 92.736) (end 161.4655 95.586) (width 0.5) (layer F.Cu) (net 13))
 (segment (start 164.4087 89.344) (end 164.4087 89.7818) (width 0.8) (layer F.Cu) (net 13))
 (segment (start 161.4805 92.71) (end 162.306 92.71) (width 0.8) (layer F.Cu) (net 13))
 (segment (start 164.4087 90.6073) (end 164.4087 89.344) (width 0.8) (layer F.Cu) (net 13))
 (segment (start 162.306 92.71) (end 164.4087 90.6073) (width 0.8) (layer F.Cu) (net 13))
 (segment (start 170.9087 89.344) (end 164.4087 89.344) (width 0.8) (layer F.Cu) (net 13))
 (segment (start 161.4655 92.725) (end 161.4805 92.71) (width 0.8) (layer F.Cu) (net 13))
 (segment (start 161.4655 95.586) (end 161.4655 92.725) (width 0.8) (layer F.Cu) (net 13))
 (segment (start 164.40602 97.836) (end 163.65602 97.086) (width 0.5) (layer F.Cu) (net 12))
 (segment (start 163.65602 97.086) (end 159.9655 97.086) (width 0.5) (layer F.Cu) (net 12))
 (segment (start 159.9655 97.086) (end 159.4655 96.586) (width 0.5) (layer F.Cu) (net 12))
 (segment (start 159.4655 96.586) (end 159.4655 90.336) (width 0.5) (layer F.Cu) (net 12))
 (segment (start 159.8655 89.936) (end 161.4655 89.936) (width 0.5) (layer F.Cu) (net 12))
 (segment (start 159.4655 90.336) (end 159.8655 89.936) (width 0.5) (layer F.Cu) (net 12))
 (segment (start 161.4655 82.136) (end 161.4655 89.936) (width 0.5) (layer F.Cu) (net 12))
 (segment (start 164.40602 97.836) (end 170.90602 97.836) (width 0.8) (layer F.Cu) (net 12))
 (segment (start 161.4655 89.895) (end 161.4805 89.91) (width 0.8) (layer F.Cu) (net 12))
 (segment (start 161.4655 82.136) (end 161.4655 89.895) (width 0.8) (layer F.Cu) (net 12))
 (segment (start 164.4015 81.086) (end 164.4015 80.264) (width 0.5) (layer F.Cu) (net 14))
 (segment (start 163.4735 79.336) (end 164.211 80.0735) (width 0.8) (layer F.Cu) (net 14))
 (segment (start 161.4655 79.336) (end 163.4735 79.336) (width 0.8) (layer F.Cu) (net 14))
 (segment (start 164.4015 80.264) (end 164.211 80.0735) (width 0.5) (layer F.Cu) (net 14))
 (segment (start 164.4015 81.086) (end 170.9015 81.086) (width 0.8) (layer F.Cu) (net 14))
 (segment (start 140.115 88.615) (end 139.615 88.615) (width 0.25) (layer F.Cu) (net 6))
 (segment (start 140.115 86.013) (end 140.115 88.615) (width 0.8) (layer F.Cu) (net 6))
 (segment (start 135.001 80.899) (end 140.115 86.013) (width 0.8) (layer F.Cu) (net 6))
 (segment (start 127.2865 77.7305) (end 127.2865 78.8995) (width 0.8) (layer F.Cu) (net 6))
 (segment (start 127.2865 78.8995) (end 129.286 80.899) (width 0.8) (layer F.Cu) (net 6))
 (segment (start 129.286 80.899) (end 135.001 80.899) (width 0.8) (layer F.Cu) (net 6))
 (segment (start 146.415 88.615) (end 140.115 88.615) (width 0.8) (layer F.Cu) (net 6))
 (segment (start 140.115 96.665) (end 137.865 96.665) (width 0.25) (layer F.Cu) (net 8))
 (segment (start 140.115 96.665) (end 138.665 96.665) (width 0.7) (layer F.Cu) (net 8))
 (segment (start 138.17 94.72) (end 140.115 96.665) (width 0.7) (layer F.Cu) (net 8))
 (segment (start 139.275 97.505) (end 140.115 96.665) (width 0.8) (layer F.Cu) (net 8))
 (segment (start 140.115 96.665) (end 139.809 96.665) (width 0.8) (layer F.Cu) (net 8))
 (segment (start 139.809 96.665) (end 137.8585 98.6155) (width 0.8) (layer F.Cu) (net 8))
 (segment (start 137.811 94.361) (end 140.115 96.665) (width 0.8) (layer F.Cu) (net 8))
 (segment (start 128.3335 94.361) (end 137.811 94.361) (width 0.8) (layer F.Cu) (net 8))
 (segment (start 127.2865 93.314) (end 128.3335 94.361) (width 0.8) (layer F.Cu) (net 8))
 (segment (start 127.2865 90.3605) (end 127.2865 93.314) (width 0.8) (layer F.Cu) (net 8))
 (segment (start 146.415 96.665) (end 140.115 96.665) (width 0.8) (layer F.Cu) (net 8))
 (segment (start 149.2 74.8) (end 149.8 74.2) (width 0.25) (layer F.Cu) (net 1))
 (segment (start 149.8 73.727) (end 149.8 74.2) (width 0.7) (layer F.Cu) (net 1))
 (segment (start 149.8 74.2) (end 157.3845 74.2) (width 0.8) (layer F.Cu) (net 1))
 (segment (start 172.4345 74.2) (end 157.3845 74.2) (width 0.7) (layer F.Cu) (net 1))
 (segment (start 174.879 76.6445) (end 172.4345 74.2) (width 0.7) (layer F.Cu) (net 1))
 (segment (start 174.879 106.299) (end 174.879 76.6445) (width 0.7) (layer F.Cu) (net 1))
 (segment (start 135.875 101.0135) (end 141.5415 106.68) (width 0.7) (layer F.Cu) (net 1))
 (segment (start 132.6515 101.0135) (end 135.875 101.0135) (width 0.7) (layer F.Cu) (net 1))
 (segment (start 159.004 106.68) (end 160.782 108.458) (width 0.7) (layer F.Cu) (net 1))
 (segment (start 172.72 108.458) (end 174.879 106.299) (width 0.7) (layer F.Cu) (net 1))
 (segment (start 160.782 108.458) (end 172.72 108.458) (width 0.7) (layer F.Cu) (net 1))
 (segment (start 131.176 101.0135) (end 132.6515 101.0135) (width 0.8) (layer F.Cu) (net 1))
 (segment (start 129.9415 99.779) (end 131.176 101.0135) (width 0.8) (layer F.Cu) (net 1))
 (segment (start 129.9415 97.9435) (end 129.9415 99.779) (width 0.8) (layer F.Cu) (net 1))
 (segment (start 129.9415 111.0835) (end 154.156 111.0835) (width 0.8) (layer F.Cu) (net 1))
 (segment (start 141.5415 106.68) (end 154.94 106.68) (width 0.7) (layer F.Cu) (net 1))
 (segment (start 154.156 111.0835) (end 154.94 110.2995) (width 0.8) (layer F.Cu) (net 1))
 (segment (start 154.94 106.68) (end 159.004 106.68) (width 0.7) (layer F.Cu) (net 1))
 (segment (start 154.94 110.2995) (end 154.94 107.061) (width 0.8) (layer F.Cu) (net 1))
 (segment (start 153.7275 92.208) (end 153.7275 93.5355) (width 0.25) (layer F.Cu) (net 15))
 (segment (start 154.1145 91.821) (end 153.7275 92.208) (width 0.25) (layer F.Cu) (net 15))
 (segment (start 152.335 84.445) (end 152.335 84.898) (width 0.25) (layer F.Cu) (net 15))
 (segment (start 152.335 84.898) (end 153.23698 85.79998) (width 0.25) (layer F.Cu) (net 15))
 (segment (start 154.1145 86.67609) (end 154.1145 91.821) (width 0.25) (layer F.Cu) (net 15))
 (segment (start 153.238391 85.799981) (end 154.1145 86.67609) (width 0.25) (layer F.Cu) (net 15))
 (segment (start 153.23698 85.79998) (end 153.238391 85.799981) (width 0.25) (layer F.Cu) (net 15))
 (segment (start 161.363 98.4885) (end 161.4655 98.386) (width 0.25) (layer F.Cu) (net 15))
 (segment (start 164.40616 101.67652) (end 170.90616 101.67652) (width 0.8) (layer F.Cu) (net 15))
 (segment (start 153.7275 93.5355) (end 153.7275 94.99) (width 0.8) (layer F.Cu) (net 15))
 (segment (start 157.1235 98.386) (end 161.4655 98.386) (width 0.8) (layer F.Cu) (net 15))
 (segment (start 153.7275 94.99) (end 157.1235 98.386) (width 0.8) (layer F.Cu) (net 15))
 (segment (start 161.4655 98.386) (end 161.4655 100.6325) (width 0.8) (layer F.Cu) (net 15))
 (segment (start 164.40616 101.67652) (end 162.50952 101.67652) (width 0.8) (layer F.Cu) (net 15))
 (segment (start 161.4655 100.6325) (end 162.50952 101.67652) (width 0.8) (layer F.Cu) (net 15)))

